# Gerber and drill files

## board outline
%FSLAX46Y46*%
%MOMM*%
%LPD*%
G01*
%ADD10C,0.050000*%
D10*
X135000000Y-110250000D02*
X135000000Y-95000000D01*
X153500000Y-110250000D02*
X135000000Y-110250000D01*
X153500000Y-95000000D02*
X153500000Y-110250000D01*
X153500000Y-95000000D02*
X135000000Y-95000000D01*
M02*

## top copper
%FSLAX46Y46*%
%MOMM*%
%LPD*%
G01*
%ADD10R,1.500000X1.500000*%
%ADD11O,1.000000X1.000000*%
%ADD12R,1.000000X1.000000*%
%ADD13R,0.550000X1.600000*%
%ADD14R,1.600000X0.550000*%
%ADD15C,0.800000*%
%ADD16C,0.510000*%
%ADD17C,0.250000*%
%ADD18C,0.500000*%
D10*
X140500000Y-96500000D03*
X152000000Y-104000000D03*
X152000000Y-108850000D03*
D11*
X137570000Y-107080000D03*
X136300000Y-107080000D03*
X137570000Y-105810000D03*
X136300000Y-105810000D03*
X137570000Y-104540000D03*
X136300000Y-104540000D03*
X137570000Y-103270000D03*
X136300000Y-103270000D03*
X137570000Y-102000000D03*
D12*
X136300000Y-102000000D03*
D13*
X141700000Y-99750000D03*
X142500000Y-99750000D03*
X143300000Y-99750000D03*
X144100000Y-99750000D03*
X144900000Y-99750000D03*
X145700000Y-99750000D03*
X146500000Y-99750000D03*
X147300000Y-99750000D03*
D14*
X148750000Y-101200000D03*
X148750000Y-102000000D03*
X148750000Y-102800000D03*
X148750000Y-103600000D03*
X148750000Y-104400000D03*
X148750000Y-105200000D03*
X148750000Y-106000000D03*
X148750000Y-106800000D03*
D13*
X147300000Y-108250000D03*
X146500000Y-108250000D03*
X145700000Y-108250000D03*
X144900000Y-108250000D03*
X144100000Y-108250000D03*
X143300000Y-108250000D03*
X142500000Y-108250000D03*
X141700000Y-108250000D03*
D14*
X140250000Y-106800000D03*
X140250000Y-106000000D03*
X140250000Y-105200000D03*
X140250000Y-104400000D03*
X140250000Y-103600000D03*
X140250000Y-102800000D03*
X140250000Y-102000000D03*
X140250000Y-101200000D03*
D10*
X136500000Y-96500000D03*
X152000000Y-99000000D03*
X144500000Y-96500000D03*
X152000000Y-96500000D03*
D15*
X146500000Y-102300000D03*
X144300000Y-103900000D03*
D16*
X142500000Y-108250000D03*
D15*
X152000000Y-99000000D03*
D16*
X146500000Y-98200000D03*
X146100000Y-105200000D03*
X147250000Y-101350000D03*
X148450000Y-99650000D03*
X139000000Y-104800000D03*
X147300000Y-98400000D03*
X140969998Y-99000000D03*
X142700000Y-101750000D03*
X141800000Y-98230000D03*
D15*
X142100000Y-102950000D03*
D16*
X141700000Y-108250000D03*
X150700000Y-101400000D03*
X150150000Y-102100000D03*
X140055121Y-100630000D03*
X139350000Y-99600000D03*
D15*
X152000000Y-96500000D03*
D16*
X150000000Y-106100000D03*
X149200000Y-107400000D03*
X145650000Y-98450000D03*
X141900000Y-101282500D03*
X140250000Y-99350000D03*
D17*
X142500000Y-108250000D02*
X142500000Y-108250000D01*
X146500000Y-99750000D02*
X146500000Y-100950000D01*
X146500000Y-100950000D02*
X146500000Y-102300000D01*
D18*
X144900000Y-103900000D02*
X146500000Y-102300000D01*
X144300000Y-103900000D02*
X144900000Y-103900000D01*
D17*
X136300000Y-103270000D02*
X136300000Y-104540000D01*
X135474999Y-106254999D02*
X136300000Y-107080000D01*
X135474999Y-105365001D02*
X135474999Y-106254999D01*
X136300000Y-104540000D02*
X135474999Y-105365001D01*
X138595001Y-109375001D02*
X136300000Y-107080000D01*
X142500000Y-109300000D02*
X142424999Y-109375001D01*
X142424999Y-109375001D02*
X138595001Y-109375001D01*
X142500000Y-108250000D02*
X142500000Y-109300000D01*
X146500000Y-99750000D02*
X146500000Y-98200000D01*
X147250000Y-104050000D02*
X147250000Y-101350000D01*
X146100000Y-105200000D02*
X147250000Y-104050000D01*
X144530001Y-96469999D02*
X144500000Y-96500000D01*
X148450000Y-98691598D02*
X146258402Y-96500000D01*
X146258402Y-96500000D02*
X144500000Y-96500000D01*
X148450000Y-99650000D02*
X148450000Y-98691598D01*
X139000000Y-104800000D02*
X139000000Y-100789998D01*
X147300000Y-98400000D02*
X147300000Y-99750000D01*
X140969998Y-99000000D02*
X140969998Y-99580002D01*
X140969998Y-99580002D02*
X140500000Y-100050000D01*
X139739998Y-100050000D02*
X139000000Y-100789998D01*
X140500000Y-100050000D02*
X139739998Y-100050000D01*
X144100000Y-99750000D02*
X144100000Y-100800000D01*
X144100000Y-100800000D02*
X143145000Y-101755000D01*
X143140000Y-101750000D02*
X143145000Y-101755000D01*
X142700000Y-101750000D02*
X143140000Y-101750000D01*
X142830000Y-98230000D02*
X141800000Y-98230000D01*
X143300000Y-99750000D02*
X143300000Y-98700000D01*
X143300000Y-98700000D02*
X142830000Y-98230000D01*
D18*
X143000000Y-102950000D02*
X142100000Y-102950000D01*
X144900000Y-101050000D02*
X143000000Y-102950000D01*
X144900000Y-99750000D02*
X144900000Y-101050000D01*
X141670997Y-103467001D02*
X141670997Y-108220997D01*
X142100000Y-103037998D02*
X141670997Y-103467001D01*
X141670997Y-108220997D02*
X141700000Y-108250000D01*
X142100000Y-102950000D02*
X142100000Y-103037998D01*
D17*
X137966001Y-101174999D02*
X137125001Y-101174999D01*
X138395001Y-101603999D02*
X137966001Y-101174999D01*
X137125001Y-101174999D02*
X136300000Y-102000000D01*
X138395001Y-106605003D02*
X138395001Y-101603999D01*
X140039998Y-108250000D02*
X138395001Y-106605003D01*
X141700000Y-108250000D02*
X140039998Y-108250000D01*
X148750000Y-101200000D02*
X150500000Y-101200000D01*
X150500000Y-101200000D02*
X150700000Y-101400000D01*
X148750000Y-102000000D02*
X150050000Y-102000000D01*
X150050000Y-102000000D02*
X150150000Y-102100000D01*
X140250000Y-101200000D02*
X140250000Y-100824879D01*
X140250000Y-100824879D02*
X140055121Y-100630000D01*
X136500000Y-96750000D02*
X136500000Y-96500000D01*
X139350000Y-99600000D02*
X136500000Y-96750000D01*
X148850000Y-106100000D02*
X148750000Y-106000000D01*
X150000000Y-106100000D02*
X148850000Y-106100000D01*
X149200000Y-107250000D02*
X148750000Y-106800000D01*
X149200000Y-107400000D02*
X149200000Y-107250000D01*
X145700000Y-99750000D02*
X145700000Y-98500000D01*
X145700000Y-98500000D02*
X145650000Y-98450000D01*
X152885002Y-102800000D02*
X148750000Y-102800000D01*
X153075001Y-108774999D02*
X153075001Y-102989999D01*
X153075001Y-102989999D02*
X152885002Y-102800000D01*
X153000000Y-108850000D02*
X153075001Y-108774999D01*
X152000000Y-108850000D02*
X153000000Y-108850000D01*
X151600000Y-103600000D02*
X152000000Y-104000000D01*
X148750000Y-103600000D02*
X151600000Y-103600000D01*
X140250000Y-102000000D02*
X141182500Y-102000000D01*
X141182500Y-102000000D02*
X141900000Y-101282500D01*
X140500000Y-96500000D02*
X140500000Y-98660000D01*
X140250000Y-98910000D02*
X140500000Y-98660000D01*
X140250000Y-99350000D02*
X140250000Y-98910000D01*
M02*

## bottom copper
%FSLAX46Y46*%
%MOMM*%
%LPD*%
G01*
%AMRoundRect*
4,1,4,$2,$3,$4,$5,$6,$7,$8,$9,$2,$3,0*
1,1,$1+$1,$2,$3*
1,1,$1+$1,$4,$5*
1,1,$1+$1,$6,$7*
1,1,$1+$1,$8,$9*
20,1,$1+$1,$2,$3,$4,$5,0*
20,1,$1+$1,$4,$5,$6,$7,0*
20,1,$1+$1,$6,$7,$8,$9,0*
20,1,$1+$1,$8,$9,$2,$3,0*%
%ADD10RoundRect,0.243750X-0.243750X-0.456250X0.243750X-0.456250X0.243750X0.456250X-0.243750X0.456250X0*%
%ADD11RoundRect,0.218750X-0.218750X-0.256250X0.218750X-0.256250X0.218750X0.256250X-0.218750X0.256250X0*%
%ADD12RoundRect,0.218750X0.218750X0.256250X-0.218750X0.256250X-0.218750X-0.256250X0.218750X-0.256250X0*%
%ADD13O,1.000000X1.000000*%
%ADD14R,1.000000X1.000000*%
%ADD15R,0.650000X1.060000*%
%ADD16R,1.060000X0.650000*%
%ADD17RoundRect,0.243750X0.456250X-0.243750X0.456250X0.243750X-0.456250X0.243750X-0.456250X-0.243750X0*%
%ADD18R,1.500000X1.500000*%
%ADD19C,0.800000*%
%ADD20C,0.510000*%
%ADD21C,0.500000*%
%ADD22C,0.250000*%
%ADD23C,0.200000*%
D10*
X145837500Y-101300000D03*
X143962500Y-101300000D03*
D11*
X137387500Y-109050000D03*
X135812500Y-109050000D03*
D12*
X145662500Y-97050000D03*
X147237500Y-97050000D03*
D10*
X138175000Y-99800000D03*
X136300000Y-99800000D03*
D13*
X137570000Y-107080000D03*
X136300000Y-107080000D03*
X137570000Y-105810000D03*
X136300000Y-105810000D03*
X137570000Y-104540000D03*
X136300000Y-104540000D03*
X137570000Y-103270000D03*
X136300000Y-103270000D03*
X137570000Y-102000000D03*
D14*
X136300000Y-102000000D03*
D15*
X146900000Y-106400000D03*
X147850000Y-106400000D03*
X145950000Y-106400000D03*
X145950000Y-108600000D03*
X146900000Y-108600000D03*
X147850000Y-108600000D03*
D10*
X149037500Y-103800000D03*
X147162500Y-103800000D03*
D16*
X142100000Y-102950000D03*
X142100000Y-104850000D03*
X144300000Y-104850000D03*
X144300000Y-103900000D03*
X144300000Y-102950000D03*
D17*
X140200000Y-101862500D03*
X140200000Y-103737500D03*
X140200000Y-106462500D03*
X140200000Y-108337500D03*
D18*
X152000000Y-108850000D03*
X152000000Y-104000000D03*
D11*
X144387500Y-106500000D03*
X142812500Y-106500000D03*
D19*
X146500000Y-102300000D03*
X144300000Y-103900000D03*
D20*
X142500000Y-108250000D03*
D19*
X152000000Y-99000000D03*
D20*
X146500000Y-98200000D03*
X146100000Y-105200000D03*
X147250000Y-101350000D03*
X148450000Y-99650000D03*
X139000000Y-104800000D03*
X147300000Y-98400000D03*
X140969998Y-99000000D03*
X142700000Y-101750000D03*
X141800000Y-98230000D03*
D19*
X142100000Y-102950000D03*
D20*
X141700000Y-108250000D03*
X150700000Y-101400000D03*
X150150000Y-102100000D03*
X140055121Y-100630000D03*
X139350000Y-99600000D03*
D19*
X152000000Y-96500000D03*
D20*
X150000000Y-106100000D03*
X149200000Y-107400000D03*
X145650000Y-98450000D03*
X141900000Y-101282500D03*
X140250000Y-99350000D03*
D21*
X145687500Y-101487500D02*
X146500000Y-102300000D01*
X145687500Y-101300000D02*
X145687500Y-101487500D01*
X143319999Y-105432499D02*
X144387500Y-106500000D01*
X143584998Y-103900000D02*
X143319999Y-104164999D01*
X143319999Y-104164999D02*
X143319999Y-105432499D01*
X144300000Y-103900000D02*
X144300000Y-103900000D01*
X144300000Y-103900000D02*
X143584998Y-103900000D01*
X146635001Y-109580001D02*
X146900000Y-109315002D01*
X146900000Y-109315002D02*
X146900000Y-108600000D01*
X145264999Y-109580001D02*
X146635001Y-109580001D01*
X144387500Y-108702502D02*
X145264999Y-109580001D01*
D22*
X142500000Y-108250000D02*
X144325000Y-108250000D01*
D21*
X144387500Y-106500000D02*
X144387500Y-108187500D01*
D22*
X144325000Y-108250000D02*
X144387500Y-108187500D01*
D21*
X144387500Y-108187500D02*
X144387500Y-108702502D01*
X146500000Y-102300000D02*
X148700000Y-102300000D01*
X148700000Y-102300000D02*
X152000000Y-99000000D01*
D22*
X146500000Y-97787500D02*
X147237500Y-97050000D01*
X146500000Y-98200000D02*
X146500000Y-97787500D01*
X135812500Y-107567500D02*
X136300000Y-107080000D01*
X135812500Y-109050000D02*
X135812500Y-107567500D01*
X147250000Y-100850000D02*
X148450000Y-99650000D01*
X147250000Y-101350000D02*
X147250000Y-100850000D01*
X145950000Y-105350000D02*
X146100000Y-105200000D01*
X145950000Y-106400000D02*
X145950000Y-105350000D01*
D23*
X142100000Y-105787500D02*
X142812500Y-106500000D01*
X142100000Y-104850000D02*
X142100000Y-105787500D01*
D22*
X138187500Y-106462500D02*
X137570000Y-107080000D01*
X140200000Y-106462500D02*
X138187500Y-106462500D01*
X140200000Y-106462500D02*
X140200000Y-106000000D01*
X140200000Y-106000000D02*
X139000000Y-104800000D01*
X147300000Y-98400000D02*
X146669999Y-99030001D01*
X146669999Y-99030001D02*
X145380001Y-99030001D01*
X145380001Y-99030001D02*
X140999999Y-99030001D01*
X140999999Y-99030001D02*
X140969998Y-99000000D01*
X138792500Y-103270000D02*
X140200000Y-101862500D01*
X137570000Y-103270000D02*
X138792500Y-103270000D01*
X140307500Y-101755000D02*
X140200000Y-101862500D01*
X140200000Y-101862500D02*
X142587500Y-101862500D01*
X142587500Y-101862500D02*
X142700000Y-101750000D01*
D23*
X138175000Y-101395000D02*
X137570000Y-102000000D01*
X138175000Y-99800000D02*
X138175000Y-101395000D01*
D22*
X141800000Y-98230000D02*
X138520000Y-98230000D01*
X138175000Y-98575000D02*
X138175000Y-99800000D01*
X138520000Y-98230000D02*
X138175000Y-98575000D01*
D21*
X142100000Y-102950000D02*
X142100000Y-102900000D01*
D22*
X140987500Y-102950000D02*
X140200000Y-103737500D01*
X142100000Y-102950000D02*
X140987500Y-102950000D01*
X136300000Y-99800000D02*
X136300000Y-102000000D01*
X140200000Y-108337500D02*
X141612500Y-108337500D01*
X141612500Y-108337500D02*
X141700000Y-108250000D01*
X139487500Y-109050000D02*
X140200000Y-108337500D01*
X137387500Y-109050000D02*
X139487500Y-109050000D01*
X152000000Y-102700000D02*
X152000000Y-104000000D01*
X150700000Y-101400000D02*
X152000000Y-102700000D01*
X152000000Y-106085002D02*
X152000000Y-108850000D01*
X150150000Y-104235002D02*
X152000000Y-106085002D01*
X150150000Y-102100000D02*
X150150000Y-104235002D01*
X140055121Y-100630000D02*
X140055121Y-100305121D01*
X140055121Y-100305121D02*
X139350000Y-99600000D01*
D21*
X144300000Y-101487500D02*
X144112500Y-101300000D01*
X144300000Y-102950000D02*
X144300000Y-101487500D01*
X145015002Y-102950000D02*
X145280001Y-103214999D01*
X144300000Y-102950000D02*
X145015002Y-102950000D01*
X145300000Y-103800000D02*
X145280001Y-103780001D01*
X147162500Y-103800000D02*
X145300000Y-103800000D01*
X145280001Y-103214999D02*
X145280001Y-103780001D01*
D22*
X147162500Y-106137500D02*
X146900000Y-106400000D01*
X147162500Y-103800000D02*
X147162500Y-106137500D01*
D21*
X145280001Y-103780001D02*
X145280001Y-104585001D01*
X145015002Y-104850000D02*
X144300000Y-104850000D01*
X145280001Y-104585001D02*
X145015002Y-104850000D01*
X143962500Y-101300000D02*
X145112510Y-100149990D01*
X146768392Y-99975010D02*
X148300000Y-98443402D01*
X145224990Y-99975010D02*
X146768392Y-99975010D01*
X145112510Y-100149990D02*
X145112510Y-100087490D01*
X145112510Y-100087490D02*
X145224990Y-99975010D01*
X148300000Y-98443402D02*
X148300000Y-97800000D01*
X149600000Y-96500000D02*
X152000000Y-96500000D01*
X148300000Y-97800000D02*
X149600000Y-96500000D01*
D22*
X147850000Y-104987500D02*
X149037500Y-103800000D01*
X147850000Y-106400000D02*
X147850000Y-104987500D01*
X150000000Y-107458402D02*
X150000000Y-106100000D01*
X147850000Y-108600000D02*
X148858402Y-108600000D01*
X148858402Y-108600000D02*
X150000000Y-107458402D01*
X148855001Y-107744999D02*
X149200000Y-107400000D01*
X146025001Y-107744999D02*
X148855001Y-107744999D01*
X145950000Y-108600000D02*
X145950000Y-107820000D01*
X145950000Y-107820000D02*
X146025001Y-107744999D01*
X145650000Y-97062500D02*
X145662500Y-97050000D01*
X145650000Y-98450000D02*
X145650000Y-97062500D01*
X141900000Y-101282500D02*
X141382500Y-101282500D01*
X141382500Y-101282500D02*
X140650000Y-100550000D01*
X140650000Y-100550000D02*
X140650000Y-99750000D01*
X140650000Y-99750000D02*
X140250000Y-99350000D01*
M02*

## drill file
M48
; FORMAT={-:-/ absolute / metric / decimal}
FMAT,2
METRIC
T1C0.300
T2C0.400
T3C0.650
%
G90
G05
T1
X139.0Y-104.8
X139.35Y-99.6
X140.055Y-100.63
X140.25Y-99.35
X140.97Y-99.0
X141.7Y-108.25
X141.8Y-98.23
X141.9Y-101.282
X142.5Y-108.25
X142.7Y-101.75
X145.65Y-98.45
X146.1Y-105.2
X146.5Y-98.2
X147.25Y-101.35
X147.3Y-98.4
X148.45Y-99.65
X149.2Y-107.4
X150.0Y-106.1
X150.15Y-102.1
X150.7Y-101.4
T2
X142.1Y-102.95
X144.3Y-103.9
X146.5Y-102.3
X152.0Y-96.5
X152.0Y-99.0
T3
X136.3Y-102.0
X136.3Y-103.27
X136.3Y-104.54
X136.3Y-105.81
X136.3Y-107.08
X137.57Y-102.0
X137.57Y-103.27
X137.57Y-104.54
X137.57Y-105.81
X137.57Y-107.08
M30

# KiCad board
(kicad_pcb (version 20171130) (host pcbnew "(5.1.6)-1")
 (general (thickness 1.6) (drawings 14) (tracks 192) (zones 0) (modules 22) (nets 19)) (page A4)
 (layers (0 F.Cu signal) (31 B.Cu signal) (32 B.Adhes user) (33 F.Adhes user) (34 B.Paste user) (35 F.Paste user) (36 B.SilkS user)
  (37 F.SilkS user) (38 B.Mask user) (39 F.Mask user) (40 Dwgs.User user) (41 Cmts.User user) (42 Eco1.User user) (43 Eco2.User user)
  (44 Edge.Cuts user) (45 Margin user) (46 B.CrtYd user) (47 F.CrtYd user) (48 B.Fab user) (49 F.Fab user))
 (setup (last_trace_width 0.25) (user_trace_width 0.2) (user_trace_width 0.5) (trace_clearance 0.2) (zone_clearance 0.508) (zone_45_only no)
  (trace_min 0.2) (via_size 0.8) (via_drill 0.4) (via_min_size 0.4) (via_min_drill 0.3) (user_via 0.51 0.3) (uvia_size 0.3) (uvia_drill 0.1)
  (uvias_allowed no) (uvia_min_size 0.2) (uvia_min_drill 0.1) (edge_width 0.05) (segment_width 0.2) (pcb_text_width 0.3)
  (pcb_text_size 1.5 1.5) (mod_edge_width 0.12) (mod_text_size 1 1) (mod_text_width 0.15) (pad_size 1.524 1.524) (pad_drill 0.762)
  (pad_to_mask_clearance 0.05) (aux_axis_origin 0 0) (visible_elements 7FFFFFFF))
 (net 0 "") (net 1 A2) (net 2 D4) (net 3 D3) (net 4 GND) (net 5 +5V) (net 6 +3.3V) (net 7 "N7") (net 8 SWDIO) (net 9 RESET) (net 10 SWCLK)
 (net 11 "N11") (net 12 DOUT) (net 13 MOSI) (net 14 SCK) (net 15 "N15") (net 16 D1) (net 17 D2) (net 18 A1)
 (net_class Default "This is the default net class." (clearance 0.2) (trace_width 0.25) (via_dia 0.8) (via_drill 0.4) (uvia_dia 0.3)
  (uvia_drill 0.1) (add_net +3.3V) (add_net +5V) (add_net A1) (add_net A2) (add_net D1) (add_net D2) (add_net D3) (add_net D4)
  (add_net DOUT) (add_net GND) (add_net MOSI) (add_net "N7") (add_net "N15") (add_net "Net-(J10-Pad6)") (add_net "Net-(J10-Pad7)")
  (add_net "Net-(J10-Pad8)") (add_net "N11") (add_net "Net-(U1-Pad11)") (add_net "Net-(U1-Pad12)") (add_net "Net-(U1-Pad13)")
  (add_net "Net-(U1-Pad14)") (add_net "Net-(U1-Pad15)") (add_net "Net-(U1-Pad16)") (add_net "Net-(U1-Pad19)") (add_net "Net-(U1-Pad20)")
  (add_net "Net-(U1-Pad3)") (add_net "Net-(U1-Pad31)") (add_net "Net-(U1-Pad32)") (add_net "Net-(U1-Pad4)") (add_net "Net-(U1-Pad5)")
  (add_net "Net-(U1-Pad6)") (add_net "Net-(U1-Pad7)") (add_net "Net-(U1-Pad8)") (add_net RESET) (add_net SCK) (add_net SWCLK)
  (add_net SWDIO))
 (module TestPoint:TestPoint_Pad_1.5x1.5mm (layer F.Cu) (at 140.5 96.5)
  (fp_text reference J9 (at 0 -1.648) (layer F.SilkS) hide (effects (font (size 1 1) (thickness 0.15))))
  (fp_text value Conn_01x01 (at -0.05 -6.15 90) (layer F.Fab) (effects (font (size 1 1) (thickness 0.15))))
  (pad 1 smd rect (at 0 0) (size 1.5 1.5) (layers F.Cu F.Mask) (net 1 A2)))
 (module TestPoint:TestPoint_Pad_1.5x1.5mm (layer F.Cu) (at 152 104)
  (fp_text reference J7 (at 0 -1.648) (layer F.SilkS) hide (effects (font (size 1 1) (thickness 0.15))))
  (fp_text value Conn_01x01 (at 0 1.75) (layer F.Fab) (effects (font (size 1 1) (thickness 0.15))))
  (pad 1 smd rect (at 0 0) (size 1.5 1.5) (layers F.Cu F.Mask) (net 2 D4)))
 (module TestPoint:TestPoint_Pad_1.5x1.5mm (layer F.Cu) (at 152 108.85)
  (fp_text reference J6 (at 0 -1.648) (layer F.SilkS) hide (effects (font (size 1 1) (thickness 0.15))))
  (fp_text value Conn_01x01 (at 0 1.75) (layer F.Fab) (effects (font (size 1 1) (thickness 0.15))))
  (pad 1 smd rect (at 0 0) (size 1.5 1.5) (layers F.Cu F.Mask) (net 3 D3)))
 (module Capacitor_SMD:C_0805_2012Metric (layer B.Cu) (at 144.9 101.3)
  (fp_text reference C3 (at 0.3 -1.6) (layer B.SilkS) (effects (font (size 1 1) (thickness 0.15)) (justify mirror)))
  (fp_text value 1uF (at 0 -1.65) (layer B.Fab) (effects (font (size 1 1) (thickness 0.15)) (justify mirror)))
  (pad 2 smd roundrect (at 0.9375 0) (size 0.975 1.4) (layers B.Cu B.Paste B.Mask) (roundrect_rratio 0.25) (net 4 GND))
  (pad 1 smd roundrect (at -0.9375 0) (size 0.975 1.4) (layers B.Cu B.Paste B.Mask) (roundrect_rratio 0.25) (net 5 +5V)))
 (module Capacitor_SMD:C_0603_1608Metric (layer B.Cu) (at 136.6 109.05)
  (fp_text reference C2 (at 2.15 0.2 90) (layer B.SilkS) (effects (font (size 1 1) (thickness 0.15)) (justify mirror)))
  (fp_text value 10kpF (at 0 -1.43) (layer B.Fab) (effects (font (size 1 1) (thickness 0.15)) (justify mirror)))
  (pad 2 smd roundrect (at 0.7875 0) (size 0.875 0.95) (layers B.Cu B.Paste B.Mask) (roundrect_rratio 0.25) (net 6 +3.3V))
  (pad 1 smd roundrect (at -0.7875 0) (size 0.875 0.95) (layers B.Cu B.Paste B.Mask) (roundrect_rratio 0.25) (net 4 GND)))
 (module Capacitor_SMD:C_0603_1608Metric (layer B.Cu) (at 146.45 97.05 180)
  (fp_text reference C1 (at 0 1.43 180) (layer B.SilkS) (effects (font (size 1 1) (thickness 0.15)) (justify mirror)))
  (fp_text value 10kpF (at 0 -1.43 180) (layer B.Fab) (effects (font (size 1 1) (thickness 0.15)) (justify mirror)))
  (pad 2 smd roundrect (at 0.7875 0 180) (size 0.875 0.95) (layers B.Cu B.Paste B.Mask) (roundrect_rratio 0.25) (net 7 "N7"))
  (pad 1 smd roundrect (at -0.7875 0 180) (size 0.875 0.95) (layers B.Cu B.Paste B.Mask) (roundrect_rratio 0.25) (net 4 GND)))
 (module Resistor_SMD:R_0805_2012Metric (layer B.Cu) (at 137.2375 99.8)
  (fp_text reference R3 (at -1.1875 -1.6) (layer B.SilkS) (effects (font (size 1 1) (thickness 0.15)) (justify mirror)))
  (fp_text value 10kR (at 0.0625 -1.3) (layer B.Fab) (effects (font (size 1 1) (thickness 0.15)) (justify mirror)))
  (pad 2 smd roundrect (at 0.9375 0) (size 0.975 1.4) (layers B.Cu B.Paste B.Mask) (roundrect_rratio 0.25) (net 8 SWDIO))
  (pad 1 smd roundrect (at -0.9375 0) (size 0.975 1.4) (layers B.Cu B.Paste B.Mask) (roundrect_rratio 0.25) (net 6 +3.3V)))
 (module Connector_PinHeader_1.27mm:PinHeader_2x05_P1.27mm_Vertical (layer F.Cu) (at 136.3 102)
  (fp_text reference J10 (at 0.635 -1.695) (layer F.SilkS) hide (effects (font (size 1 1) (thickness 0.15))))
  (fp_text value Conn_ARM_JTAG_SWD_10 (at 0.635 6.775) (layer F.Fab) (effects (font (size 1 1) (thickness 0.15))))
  (pad 10 thru_hole oval (at 1.27 5.08) (size 1 1) (drill 0.65) (layers *.Cu *.Mask) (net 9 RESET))
  (pad 9 thru_hole oval (at 0 5.08) (size 1 1) (drill 0.65) (layers *.Cu *.Mask) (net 4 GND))
  (pad 8 thru_hole oval (at 1.27 3.81) (size 1 1) (drill 0.65) (layers *.Cu *.Mask))
  (pad 7 thru_hole oval (at 0 3.81) (size 1 1) (drill 0.65) (layers *.Cu *.Mask))
  (pad 6 thru_hole oval (at 1.27 2.54) (size 1 1) (drill 0.65) (layers *.Cu *.Mask))
  (pad 5 thru_hole oval (at 0 2.54) (size 1 1) (drill 0.65) (layers *.Cu *.Mask) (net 4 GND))
  (pad 4 thru_hole oval (at 1.27 1.27) (size 1 1) (drill 0.65) (layers *.Cu *.Mask) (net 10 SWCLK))
  (pad 3 thru_hole oval (at 0 1.27) (size 1 1) (drill 0.65) (layers *.Cu *.Mask) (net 4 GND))
  (pad 2 thru_hole oval (at 1.27 0) (size 1 1) (drill 0.65) (layers *.Cu *.Mask) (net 8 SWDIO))
  (pad 1 thru_hole rect (at 0 0) (size 1 1) (drill 0.65) (layers *.Cu *.Mask) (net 6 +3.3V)))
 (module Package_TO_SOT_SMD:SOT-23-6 (layer B.Cu) (at 146.9 107.5 90)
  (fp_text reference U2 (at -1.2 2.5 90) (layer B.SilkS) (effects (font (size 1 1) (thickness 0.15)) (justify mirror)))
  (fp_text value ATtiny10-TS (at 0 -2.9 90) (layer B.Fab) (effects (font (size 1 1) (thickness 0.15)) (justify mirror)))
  (pad 5 smd rect (at 1.1 0 90) (size 1.06 0.65) (layers B.Cu B.Paste B.Mask) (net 5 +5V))
  (pad 6 smd rect (at 1.1 0.95 90) (size 1.06 0.65) (layers B.Cu B.Paste B.Mask) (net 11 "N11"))
  (pad 4 smd rect (at 1.1 -0.95 90) (size 1.06 0.65) (layers B.Cu B.Paste B.Mask) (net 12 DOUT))
  (pad 3 smd rect (at -1.1 -0.95 90) (size 1.06 0.65) (layers B.Cu B.Paste B.Mask) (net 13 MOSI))
  (pad 2 smd rect (at -1.1 0 90) (size 1.06 0.65) (layers B.Cu B.Paste B.Mask) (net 4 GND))
  (pad 1 smd rect (at -1.1 0.95 90) (size 1.06 0.65) (layers B.Cu B.Paste B.Mask) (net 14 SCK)))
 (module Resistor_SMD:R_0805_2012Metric (layer B.Cu) (at 148.1 103.8)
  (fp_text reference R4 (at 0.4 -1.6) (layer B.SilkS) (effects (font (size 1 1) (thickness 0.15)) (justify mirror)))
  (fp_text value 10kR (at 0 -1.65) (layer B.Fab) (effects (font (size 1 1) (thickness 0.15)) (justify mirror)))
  (pad 2 smd roundrect (at 0.9375 0) (size 0.975 1.4) (layers B.Cu B.Paste B.Mask) (roundrect_rratio 0.25) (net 11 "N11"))
  (pad 1 smd roundrect (at -0.9375 0) (size 0.975 1.4) (layers B.Cu B.Paste B.Mask) (roundrect_rratio 0.25) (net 5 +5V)))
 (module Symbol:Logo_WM (layer F.Cu) (at 137.8 99.1)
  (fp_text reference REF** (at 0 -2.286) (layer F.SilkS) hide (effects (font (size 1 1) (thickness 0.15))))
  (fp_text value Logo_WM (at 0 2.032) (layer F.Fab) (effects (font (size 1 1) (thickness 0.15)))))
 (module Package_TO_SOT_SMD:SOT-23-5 (layer B.Cu) (at 143.2 103.9 180)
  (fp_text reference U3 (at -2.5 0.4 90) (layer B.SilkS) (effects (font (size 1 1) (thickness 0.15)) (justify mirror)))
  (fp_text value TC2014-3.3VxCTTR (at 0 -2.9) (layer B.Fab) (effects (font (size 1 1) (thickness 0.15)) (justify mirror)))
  (pad 5 smd rect (at 1.1 0.95 180) (size 1.06 0.65) (layers B.Cu B.Paste B.Mask) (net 6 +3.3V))
  (pad 4 smd rect (at 1.1 -0.95 180) (size 1.06 0.65) (layers B.Cu B.Paste B.Mask) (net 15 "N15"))
  (pad 3 smd rect (at -1.1 -0.95 180) (size 1.06 0.65) (layers B.Cu B.Paste B.Mask) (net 5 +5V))
  (pad 2 smd rect (at -1.1 0 180) (size 1.06 0.65) (layers B.Cu B.Paste B.Mask) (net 4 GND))
  (pad 1 smd rect (at -1.1 0.95 180) (size 1.06 0.65) (layers B.Cu B.Paste B.Mask) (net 5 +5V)))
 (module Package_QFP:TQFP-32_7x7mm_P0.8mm (layer F.Cu) (at 144.5 104)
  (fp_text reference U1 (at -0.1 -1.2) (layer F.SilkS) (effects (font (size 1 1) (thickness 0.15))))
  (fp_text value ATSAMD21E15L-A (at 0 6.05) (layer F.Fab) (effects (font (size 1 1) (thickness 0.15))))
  (pad 32 smd rect (at -2.8 -4.25 90) (size 1.6 0.55) (layers F.Cu F.Paste F.Mask))
  (pad 31 smd rect (at -2 -4.25 90) (size 1.6 0.55) (layers F.Cu F.Paste F.Mask))
  (pad 30 smd rect (at -1.2 -4.25 90) (size 1.6 0.55) (layers F.Cu F.Paste F.Mask) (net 8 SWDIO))
  (pad 29 smd rect (at -0.4 -4.25 90) (size 1.6 0.55) (layers F.Cu F.Paste F.Mask) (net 10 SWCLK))
  (pad 28 smd rect (at 0.4 -4.25 90) (size 1.6 0.55) (layers F.Cu F.Paste F.Mask) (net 6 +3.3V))
  (pad 27 smd rect (at 1.2 -4.25 90) (size 1.6 0.55) (layers F.Cu F.Paste F.Mask) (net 7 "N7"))
  (pad 26 smd rect (at 2 -4.25 90) (size 1.6 0.55) (layers F.Cu F.Paste F.Mask) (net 4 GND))
  (pad 25 smd rect (at 2.8 -4.25 90) (size 1.6 0.55) (layers F.Cu F.Paste F.Mask) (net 9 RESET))
  (pad 24 smd rect (at 4.25 -2.8) (size 1.6 0.55) (layers F.Cu F.Paste F.Mask) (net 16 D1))
  (pad 23 smd rect (at 4.25 -2) (size 1.6 0.55) (layers F.Cu F.Paste F.Mask) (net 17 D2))
  (pad 22 smd rect (at 4.25 -1.2) (size 1.6 0.55) (layers F.Cu F.Paste F.Mask) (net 3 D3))
  (pad 21 smd rect (at 4.25 -0.4) (size 1.6 0.55) (layers F.Cu F.Paste F.Mask) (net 2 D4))
  (pad 20 smd rect (at 4.25 0.4) (size 1.6 0.55) (layers F.Cu F.Paste F.Mask))
  (pad 19 smd rect (at 4.25 1.2) (size 1.6 0.55) (layers F.Cu F.Paste F.Mask))
  (pad 18 smd rect (at 4.25 2) (size 1.6 0.55) (layers F.Cu F.Paste F.Mask) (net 14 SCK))
  (pad 17 smd rect (at 4.25 2.8) (size 1.6 0.55) (layers F.Cu F.Paste F.Mask) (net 13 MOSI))
  (pad 16 smd rect (at 2.8 4.25 90) (size 1.6 0.55) (layers F.Cu F.Paste F.Mask))
  (pad 15 smd rect (at 2 4.25 90) (size 1.6 0.55) (layers F.Cu F.Paste F.Mask))
  (pad 14 smd rect (at 1.2 4.25 90) (size 1.6 0.55) (layers F.Cu F.Paste F.Mask))
  (pad 13 smd rect (at 0.4 4.25 90) (size 1.6 0.55) (layers F.Cu F.Paste F.Mask))
  (pad 12 smd rect (at -0.4 4.25 90) (size 1.6 0.55) (layers F.Cu F.Paste F.Mask))
  (pad 11 smd rect (at -1.2 4.25 90) (size 1.6 0.55) (layers F.Cu F.Paste F.Mask))
  (pad 10 smd rect (at -2 4.25 90) (size 1.6 0.55) (layers F.Cu F.Paste F.Mask) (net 4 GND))
  (pad 9 smd rect (at -2.8 4.25 90) (size 1.6 0.55) (layers F.Cu F.Paste F.Mask) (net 6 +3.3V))
  (pad 8 smd rect (at -4.25 2.8) (size 1.6 0.55) (layers F.Cu F.Paste F.Mask))
  (pad 7 smd rect (at -4.25 2) (size 1.6 0.55) (layers F.Cu F.Paste F.Mask))
  (pad 6 smd rect (at -4.25 1.2) (size 1.6 0.55) (layers F.Cu F.Paste F.Mask))
  (pad 5 smd rect (at -4.25 0.4) (size 1.6 0.55) (layers F.Cu F.Paste F.Mask))
  (pad 4 smd rect (at -4.25 -0.4) (size 1.6 0.55) (layers F.Cu F.Paste F.Mask))
  (pad 3 smd rect (at -4.25 -1.2) (size 1.6 0.55) (layers F.Cu F.Paste F.Mask))
  (pad 2 smd rect (at -4.25 -2) (size 1.6 0.55) (layers F.Cu F.Paste F.Mask) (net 1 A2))
  (pad 1 smd rect (at -4.25 -2.8) (size 1.6 0.55) (layers F.Cu F.Paste F.Mask) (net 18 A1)))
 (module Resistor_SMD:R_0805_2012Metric (layer B.Cu) (at 140.2 102.8 90)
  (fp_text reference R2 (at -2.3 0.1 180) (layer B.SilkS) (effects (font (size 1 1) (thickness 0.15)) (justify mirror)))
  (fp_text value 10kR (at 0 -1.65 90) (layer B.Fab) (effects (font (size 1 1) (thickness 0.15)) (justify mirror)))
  (pad 2 smd roundrect (at 0.9375 0 90) (size 0.975 1.4) (layers B.Cu B.Paste B.Mask) (roundrect_rratio 0.25) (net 10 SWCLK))
  (pad 1 smd roundrect (at -0.9375 0 90) (size 0.975 1.4) (layers B.Cu B.Paste B.Mask) (roundrect_rratio 0.25) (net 6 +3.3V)))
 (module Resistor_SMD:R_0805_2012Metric (layer B.Cu) (at 140.2 107.4 90)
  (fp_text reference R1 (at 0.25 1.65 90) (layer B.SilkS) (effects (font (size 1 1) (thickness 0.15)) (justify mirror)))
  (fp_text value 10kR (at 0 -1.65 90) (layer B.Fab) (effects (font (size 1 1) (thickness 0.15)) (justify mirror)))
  (pad 2 smd roundrect (at 0.9375 0 90) (size 0.975 1.4) (layers B.Cu B.Paste B.Mask) (roundrect_rratio 0.25) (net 9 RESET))
  (pad 1 smd roundrect (at -0.9375 0 90) (size 0.975 1.4) (layers B.Cu B.Paste B.Mask) (roundrect_rratio 0.25) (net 6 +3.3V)))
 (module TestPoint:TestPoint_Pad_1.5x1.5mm (layer F.Cu) (at 136.5 96.5)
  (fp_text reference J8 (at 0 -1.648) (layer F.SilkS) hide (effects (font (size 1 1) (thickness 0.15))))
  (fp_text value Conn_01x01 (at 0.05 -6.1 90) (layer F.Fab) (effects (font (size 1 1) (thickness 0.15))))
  (pad 1 smd rect (at 0 0) (size 1.5 1.5) (layers F.Cu F.Mask) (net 18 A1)))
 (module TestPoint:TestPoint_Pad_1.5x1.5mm (layer B.Cu) (at 152 108.85)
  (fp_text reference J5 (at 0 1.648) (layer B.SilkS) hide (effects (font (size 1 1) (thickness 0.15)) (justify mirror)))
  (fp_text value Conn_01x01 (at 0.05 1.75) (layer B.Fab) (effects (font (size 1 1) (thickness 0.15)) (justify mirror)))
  (pad 1 smd rect (at 0 0) (size 1.5 1.5) (layers B.Cu B.Mask) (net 17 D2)))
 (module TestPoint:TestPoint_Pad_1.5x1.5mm (layer B.Cu) (at 152 104)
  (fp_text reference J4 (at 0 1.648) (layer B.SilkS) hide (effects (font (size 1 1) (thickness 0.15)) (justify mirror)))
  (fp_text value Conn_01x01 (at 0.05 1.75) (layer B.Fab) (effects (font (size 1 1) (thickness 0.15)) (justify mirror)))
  (pad 1 smd rect (at 0 0) (size 1.5 1.5) (layers B.Cu B.Mask) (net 16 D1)))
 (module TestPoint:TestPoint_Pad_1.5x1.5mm (layer F.Cu) (at 152 99)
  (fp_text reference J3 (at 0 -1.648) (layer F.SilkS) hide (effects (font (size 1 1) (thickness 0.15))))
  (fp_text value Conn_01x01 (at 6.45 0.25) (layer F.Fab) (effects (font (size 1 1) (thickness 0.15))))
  (pad 1 smd rect (at 0 0) (size 1.5 1.5) (layers F.Cu F.Mask) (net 4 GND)))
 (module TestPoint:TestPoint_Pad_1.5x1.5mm (layer F.Cu) (at 144.5 96.5)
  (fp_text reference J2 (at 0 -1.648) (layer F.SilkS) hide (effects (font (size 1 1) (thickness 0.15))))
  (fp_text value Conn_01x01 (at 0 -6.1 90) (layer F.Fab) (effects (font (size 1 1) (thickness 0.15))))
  (pad 1 smd rect (at 0 0) (size 1.5 1.5) (layers F.Cu F.Mask) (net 12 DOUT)))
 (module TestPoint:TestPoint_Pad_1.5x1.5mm (layer F.Cu) (at 152 96.5)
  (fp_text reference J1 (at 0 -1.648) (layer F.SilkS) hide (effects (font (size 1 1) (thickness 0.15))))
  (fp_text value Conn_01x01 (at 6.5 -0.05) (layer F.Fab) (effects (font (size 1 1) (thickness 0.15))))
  (pad 1 smd rect (at 0 0) (size 1.5 1.5) (layers F.Cu F.Mask) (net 5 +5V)))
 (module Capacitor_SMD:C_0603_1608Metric (layer B.Cu) (at 143.6 106.5)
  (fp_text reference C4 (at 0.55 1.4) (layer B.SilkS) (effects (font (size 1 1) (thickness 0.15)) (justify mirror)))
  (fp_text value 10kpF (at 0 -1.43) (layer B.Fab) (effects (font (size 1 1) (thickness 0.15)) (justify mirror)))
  (pad 2 smd roundrect (at 0.7875 0) (size 0.875 0.95) (layers B.Cu B.Paste B.Mask) (roundrect_rratio 0.25) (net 4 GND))
  (pad 1 smd roundrect (at -0.7875 0) (size 0.875 0.95) (layers B.Cu B.Paste B.Mask) (roundrect_rratio 0.25) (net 15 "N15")))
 (gr_line (start 135 110.25) (end 135 95) (layer Edge.Cuts) (width 0.05))
 (gr_line (start 153.5 110.25) (end 135 110.25) (layer Edge.Cuts) (width 0.05))
 (gr_line (start 153.5 95) (end 153.5 110.25) (layer Edge.Cuts) (width 0.05))
 (gr_line (start 153.5 95) (end 135 95) (layer Edge.Cuts) (width 0.05))
 (segment (start 142.5 108.25) (end 142.5 108.25) (width 0.25) (layer F.Cu) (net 4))
 (segment (start 146.5 99.75) (end 146.5 100.95) (width 0.25) (layer F.Cu) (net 4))
 (segment (start 145.6875 101.4875) (end 146.5 102.3) (width 0.5) (layer B.Cu) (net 4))
 (segment (start 145.6875 101.3) (end 145.6875 101.4875) (width 0.5) (layer B.Cu) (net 4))
 (via (at 146.5 102.3) (size 0.8) (drill 0.4) (layers F.Cu B.Cu) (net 4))
 (segment (start 146.5 100.95) (end 146.5 102.3) (width 0.25) (layer F.Cu) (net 4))
 (segment (start 143.319999 105.432499) (end 144.3875 106.5) (width 0.5) (layer B.Cu) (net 4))
 (segment (start 143.584998 103.9) (end 143.319999 104.164999) (width 0.5) (layer B.Cu) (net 4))
 (segment (start 143.319999 104.164999) (end 143.319999 105.432499) (width 0.5) (layer B.Cu) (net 4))
 (segment (start 144.3 103.9) (end 144.3 103.9) (width 0.5) (layer B.Cu) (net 4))
 (segment (start 144.3 103.9) (end 143.584998 103.9) (width 0.5) (layer B.Cu) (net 4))
 (via (at 144.3 103.9) (size 0.8) (drill 0.4) (layers F.Cu B.Cu) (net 4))
 (segment (start 144.9 103.9) (end 146.5 102.3) (width 0.5) (layer F.Cu) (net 4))
 (segment (start 144.3 103.9) (end 144.9 103.9) (width 0.5) (layer F.Cu) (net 4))
 (segment (start 146.635001 109.580001) (end 146.9 109.315002) (width 0.5) (layer B.Cu) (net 4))
 (segment (start 146.9 109.315002) (end 146.9 108.6) (width 0.5) (layer B.Cu) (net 4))
 (segment (start 145.264999 109.580001) (end 146.635001 109.580001) (width 0.5) (layer B.Cu) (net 4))
 (segment (start 144.3875 108.702502) (end 145.264999 109.580001) (width 0.5) (layer B.Cu) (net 4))
 (via (at 142.5 108.25) (size 0.51) (drill 0.3) (layers F.Cu B.Cu) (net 4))
 (segment (start 142.5 108.25) (end 144.325 108.25) (width 0.25) (layer B.Cu) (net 4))
 (segment (start 144.3875 106.5) (end 144.3875 108.1875) (width 0.5) (layer B.Cu) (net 4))
 (segment (start 144.325 108.25) (end 144.3875 108.1875) (width 0.25) (layer B.Cu) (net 4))
 (segment (start 144.3875 108.1875) (end 144.3875 108.702502) (width 0.5) (layer B.Cu) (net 4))
 (segment (start 136.3 103.27) (end 136.3 104.54) (width 0.25) (layer F.Cu) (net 4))
 (segment (start 135.474999 106.254999) (end 136.3 107.08) (width 0.25) (layer F.Cu) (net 4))
 (segment (start 135.474999 105.365001) (end 135.474999 106.254999) (width 0.25) (layer F.Cu) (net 4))
 (segment (start 136.3 104.54) (end 135.474999 105.365001) (width 0.25) (layer F.Cu) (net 4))
 (segment (start 138.595001 109.375001) (end 136.3 107.08) (width 0.25) (layer F.Cu) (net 4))
 (segment (start 142.5 109.3) (end 142.424999 109.375001) (width 0.25) (layer F.Cu) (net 4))
 (segment (start 142.424999 109.375001) (end 138.595001 109.375001) (width 0.25) (layer F.Cu) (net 4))
 (segment (start 142.5 108.25) (end 142.5 109.3) (width 0.25) (layer F.Cu) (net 4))
 (via (at 152 99) (size 0.8) (drill 0.4) (layers F.Cu B.Cu) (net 4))
 (segment (start 146.5 102.3) (end 148.7 102.3) (width 0.5) (layer B.Cu) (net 4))
 (segment (start 148.7 102.3) (end 152 99) (width 0.5) (layer B.Cu) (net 4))
 (via (at 146.5 98.2) (size 0.51) (drill 0.3) (layers F.Cu B.Cu) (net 4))
 (segment (start 146.5 99.75) (end 146.5 98.2) (width 0.25) (layer F.Cu) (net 4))
 (segment (start 146.5 97.7875) (end 147.2375 97.05) (width 0.25) (layer B.Cu) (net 4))
 (segment (start 146.5 98.2) (end 146.5 97.7875) (width 0.25) (layer B.Cu) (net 4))
 (segment (start 135.8125 107.5675) (end 136.3 107.08) (width 0.25) (layer B.Cu) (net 4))
 (segment (start 135.8125 109.05) (end 135.8125 107.5675) (width 0.25) (layer B.Cu) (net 4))
 (via (at 146.1 105.2) (size 0.51) (drill 0.3) (layers F.Cu B.Cu) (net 12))
 (via (at 147.25 101.35) (size 0.51) (drill 0.3) (layers F.Cu B.Cu) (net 12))
 (via (at 148.45 99.65) (size 0.51) (drill 0.3) (layers F.Cu B.Cu) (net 12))
 (segment (start 147.25 104.05) (end 147.25 101.35) (width 0.25) (layer F.Cu) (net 12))
 (segment (start 147.25 100.85) (end 148.45 99.65) (width 0.25) (layer B.Cu) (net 12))
 (segment (start 147.25 101.35) (end 147.25 100.85) (width 0.25) (layer B.Cu) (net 12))
 (segment (start 146.1 105.2) (end 147.25 104.05) (width 0.25) (layer F.Cu) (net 12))
 (segment (start 144.530001 96.469999) (end 144.5 96.5) (width 0.25) (layer F.Cu) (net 12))
 (segment (start 145.95 105.35) (end 146.1 105.2) (width 0.25) (layer B.Cu) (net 12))
 (segment (start 145.95 106.4) (end 145.95 105.35) (width 0.25) (layer B.Cu) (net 12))
 (segment (start 148.45 98.691598) (end 146.258402 96.5) (width 0.25) (layer F.Cu) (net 12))
 (segment (start 146.258402 96.5) (end 144.5 96.5) (width 0.25) (layer F.Cu) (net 12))
 (segment (start 148.45 99.65) (end 148.45 98.691598) (width 0.25) (layer F.Cu) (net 12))
 (segment (start 142.1 105.7875) (end 142.8125 106.5) (width 0.2) (layer B.Cu) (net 15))
 (segment (start 142.1 104.85) (end 142.1 105.7875) (width 0.2) (layer B.Cu) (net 15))
 (segment (start 138.1875 106.4625) (end 137.57 107.08) (width 0.25) (layer B.Cu) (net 9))
 (segment (start 140.2 106.4625) (end 138.1875 106.4625) (width 0.25) (layer B.Cu) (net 9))
 (via (at 139 104.8) (size 0.51) (drill 0.3) (layers F.Cu B.Cu) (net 9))
 (segment (start 140.2 106.4625) (end 140.2 106) (width 0.25) (layer B.Cu) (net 9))
 (segment (start 140.2 106) (end 139 104.8) (width 0.25) (layer B.Cu) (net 9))
 (segment (start 139 104.8) (end 139 100.789998) (width 0.25) (layer F.Cu) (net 9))
 (via (at 147.3 98.4) (size 0.51) (drill 0.3) (layers F.Cu B.Cu) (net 9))
 (segment (start 147.3 98.4) (end 147.3 99.75) (width 0.25) (layer F.Cu) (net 9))
 (segment (start 147.3 98.4) (end 146.669999 99.030001) (width 0.25) (layer B.Cu) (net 9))
 (segment (start 146.669999 99.030001) (end 145.380001 99.030001) (width 0.25) (layer B.Cu) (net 9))
 (segment (start 145.380001 99.030001) (end 140.999999 99.030001) (width 0.25) (layer B.Cu) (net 9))
 (via (at 140.969998 99) (size 0.51) (drill 0.3) (layers F.Cu B.Cu) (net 9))
 (segment (start 140.999999 99.030001) (end 140.969998 99) (width 0.25) (layer B.Cu) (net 9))
 (segment (start 140.969998 99) (end 140.969998 99.580002) (width 0.25) (layer F.Cu) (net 9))
 (segment (start 140.969998 99.580002) (end 140.5 100.05) (width 0.25) (layer F.Cu) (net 9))
 (segment (start 139.739998 100.05) (end 139 100.789998) (width 0.25) (layer F.Cu) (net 9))
 (segment (start 140.5 100.05) (end 139.739998 100.05) (width 0.25) (layer F.Cu) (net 9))
 (segment (start 138.7925 103.27) (end 140.2 101.8625) (width 0.25) (layer B.Cu) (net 10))
 (segment (start 137.57 103.27) (end 138.7925 103.27) (width 0.25) (layer B.Cu) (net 10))
 (segment (start 144.1 99.75) (end 144.1 100.8) (width 0.25) (layer F.Cu) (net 10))
 (segment (start 144.1 100.8) (end 143.145 101.755) (width 0.25) (layer F.Cu) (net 10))
 (segment (start 140.3075 101.755) (end 140.2 101.8625) (width 0.25) (layer B.Cu) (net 10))
 (via (at 142.7 101.75) (size 0.51) (drill 0.3) (layers F.Cu B.Cu) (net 10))
 (segment (start 140.2 101.8625) (end 142.5875 101.8625) (width 0.25) (layer B.Cu) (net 10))
 (segment (start 142.5875 101.8625) (end 142.7 101.75) (width 0.25) (layer B.Cu) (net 10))
 (segment (start 143.14 101.75) (end 143.145 101.755) (width 0.25) (layer F.Cu) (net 10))
 (segment (start 142.7 101.75) (end 143.14 101.75) (width 0.25) (layer F.Cu) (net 10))
 (segment (start 138.175 101.395) (end 137.57 102) (width 0.2) (layer B.Cu) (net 8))
 (segment (start 138.175 99.8) (end 138.175 101.395) (width 0.2) (layer B.Cu) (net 8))
 (segment (start 142.83 98.23) (end 141.8 98.23) (width 0.25) (layer F.Cu) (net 8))
 (segment (start 143.3 99.75) (end 143.3 98.7) (width 0.25) (layer F.Cu) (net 8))
 (via (at 141.8 98.23) (size 0.51) (drill 0.3) (layers F.Cu B.Cu) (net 8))
 (segment (start 143.3 98.7) (end 142.83 98.23) (width 0.25) (layer F.Cu) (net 8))
 (segment (start 141.8 98.23) (end 138.52 98.23) (width 0.25) (layer B.Cu) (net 8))
 (segment (start 138.175 98.575) (end 138.175 99.8) (width 0.25) (layer B.Cu) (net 8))
 (segment (start 138.52 98.23) (end 138.175 98.575) (width 0.25) (layer B.Cu) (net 8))
 (segment (start 143 102.95) (end 142.1 102.95) (width 0.5) (layer F.Cu) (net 6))
 (via (at 142.1 102.95) (size 0.8) (drill 0.4) (layers F.Cu B.Cu) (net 6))
 (segment (start 144.9 101.05) (end 143 102.95) (width 0.5) (layer F.Cu) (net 6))
 (segment (start 144.9 99.75) (end 144.9 101.05) (width 0.5) (layer F.Cu) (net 6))
 (segment (start 141.670997 103.467001) (end 141.670997 108.220997) (width 0.5) (layer F.Cu) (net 6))
 (segment (start 142.1 103.037998) (end 141.670997 103.467001) (width 0.5) (layer F.Cu) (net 6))
 (segment (start 141.670997 108.220997) (end 141.7 108.25) (width 0.5) (layer F.Cu) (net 6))
 (segment (start 142.1 102.95) (end 142.1 103.037998) (width 0.5) (layer F.Cu) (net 6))
 (segment (start 142.1 102.95) (end 142.1 102.9) (width 0.5) (layer B.Cu) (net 6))
 (segment (start 140.9875 102.95) (end 140.2 103.7375) (width 0.25) (layer B.Cu) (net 6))
 (segment (start 142.1 102.95) (end 140.9875 102.95) (width 0.25) (layer B.Cu) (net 6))
 (segment (start 136.3 99.8) (end 136.3 102) (width 0.25) (layer B.Cu) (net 6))
 (via (at 141.7 108.25) (size 0.51) (drill 0.3) (layers F.Cu B.Cu) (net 6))
 (segment (start 140.2 108.3375) (end 141.6125 108.3375) (width 0.25) (layer B.Cu) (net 6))
 (segment (start 141.6125 108.3375) (end 141.7 108.25) (width 0.25) (layer B.Cu) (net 6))
 (segment (start 137.966001 101.174999) (end 137.125001 101.174999) (width 0.25) (layer F.Cu) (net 6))
 (segment (start 138.395001 101.603999) (end 137.966001 101.174999) (width 0.25) (layer F.Cu) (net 6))
 (segment (start 137.125001 101.174999) (end 136.3 102) (width 0.25) (layer F.Cu) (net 6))
 (segment (start 138.395001 106.605003) (end 138.395001 101.603999) (width 0.25) (layer F.Cu) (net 6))
 (segment (start 140.039998 108.25) (end 138.395001 106.605003) (width 0.25) (layer F.Cu) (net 6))
 (segment (start 141.7 108.25) (end 140.039998 108.25) (width 0.25) (layer F.Cu) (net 6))
 (segment (start 139.4875 109.05) (end 140.2 108.3375) (width 0.25) (layer B.Cu) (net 6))
 (segment (start 137.3875 109.05) (end 139.4875 109.05) (width 0.25) (layer B.Cu) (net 6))
 (segment (start 148.75 101.2) (end 150.5 101.2) (width 0.25) (layer F.Cu) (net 16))
 (via (at 150.7 101.4) (size 0.51) (drill 0.3) (layers F.Cu B.Cu) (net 16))
 (segment (start 150.5 101.2) (end 150.7 101.4) (width 0.25) (layer F.Cu) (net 16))
 (segment (start 152 102.7) (end 152 104) (width 0.25) (layer B.Cu) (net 16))
 (segment (start 150.7 101.4) (end 152 102.7) (width 0.25) (layer B.Cu) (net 16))
 (via (at 150.15 102.1) (size 0.51) (drill 0.3) (layers F.Cu B.Cu) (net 17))
 (segment (start 148.75 102) (end 150.05 102) (width 0.25) (layer F.Cu) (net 17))
 (segment (start 150.05 102) (end 150.15 102.1) (width 0.25) (layer F.Cu) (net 17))
 (segment (start 152 106.085002) (end 152 108.85) (width 0.25) (layer B.Cu) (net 17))
 (segment (start 150.15 104.235002) (end 152 106.085002) (width 0.25) (layer B.Cu) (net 17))
 (segment (start 150.15 102.1) (end 150.15 104.235002) (width 0.25) (layer B.Cu) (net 17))
 (via (at 140.055121 100.63) (size 0.51) (drill 0.3) (layers F.Cu B.Cu) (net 18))
 (segment (start 140.25 101.2) (end 140.25 100.824879) (width 0.25) (layer F.Cu) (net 18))
 (segment (start 140.25 100.824879) (end 140.055121 100.63) (width 0.25) (layer F.Cu) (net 18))
 (via (at 139.35 99.6) (size 0.51) (drill 0.3) (layers F.Cu B.Cu) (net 18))
 (segment (start 140.055121 100.63) (end 140.055121 100.305121) (width 0.25) (layer B.Cu) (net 18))
 (segment (start 140.055121 100.305121) (end 139.35 99.6) (width 0.25) (layer B.Cu) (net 18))
 (segment (start 136.5 96.75) (end 136.5 96.5) (width 0.25) (layer F.Cu) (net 18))
 (segment (start 139.35 99.6) (end 136.5 96.75) (width 0.25) (layer F.Cu) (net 18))
 (segment (start 144.3 101.4875) (end 144.1125 101.3) (width 0.5) (layer B.Cu) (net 5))
 (segment (start 144.3 102.95) (end 144.3 101.4875) (width 0.5) (layer B.Cu) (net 5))
 (segment (start 145.015002 102.95) (end 145.280001 103.214999) (width 0.5) (layer B.Cu) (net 5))
 (segment (start 144.3 102.95) (end 145.015002 102.95) (width 0.5) (layer B.Cu) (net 5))
 (segment (start 145.3 103.8) (end 145.280001 103.780001) (width 0.5) (layer B.Cu) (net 5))
 (segment (start 147.1625 103.8) (end 145.3 103.8) (width 0.5) (layer B.Cu) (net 5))
 (segment (start 145.280001 103.214999) (end 145.280001 103.780001) (width 0.5) (layer B.Cu) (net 5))
 (segment (start 147.1625 106.1375) (end 146.9 106.4) (width 0.25) (layer B.Cu) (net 5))
 (segment (start 147.1625 103.8) (end 147.1625 106.1375) (width 0.25) (layer B.Cu) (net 5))
 (segment (start 145.280001 103.780001) (end 145.280001 104.585001) (width 0.5) (layer B.Cu) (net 5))
 (segment (start 145.015002 104.85) (end 144.3 104.85) (width 0.5) (layer B.Cu) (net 5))
 (segment (start 145.280001 104.585001) (end 145.015002 104.85) (width 0.5) (layer B.Cu) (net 5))
 (via (at 152 96.5) (size 0.8) (drill 0.4) (layers F.Cu B.Cu) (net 5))
 (segment (start 143.9625 101.3) (end 145.11251 100.14999) (width 0.5) (layer B.Cu) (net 5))
 (segment (start 146.768392 99.97501) (end 148.3 98.443402) (width 0.5) (layer B.Cu) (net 5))
 (segment (start 145.22499 99.97501) (end 146.768392 99.97501) (width 0.5) (layer B.Cu) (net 5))
 (segment (start 145.11251 100.14999) (end 145.11251 100.08749) (width 0.5) (layer B.Cu) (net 5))
 (segment (start 145.11251 100.08749) (end 145.22499 99.97501) (width 0.5) (layer B.Cu) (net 5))
 (segment (start 148.3 98.443402) (end 148.3 97.8) (width 0.5) (layer B.Cu) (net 5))
 (segment (start 149.6 96.5) (end 152 96.5) (width 0.5) (layer B.Cu) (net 5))
 (segment (start 148.3 97.8) (end 149.6 96.5) (width 0.5) (layer B.Cu) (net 5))
 (segment (start 147.85 104.9875) (end 149.0375 103.8) (width 0.25) (layer B.Cu) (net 11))
 (segment (start 147.85 106.4) (end 147.85 104.9875) (width 0.25) (layer B.Cu) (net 11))
 (via (at 150 106.1) (size 0.51) (drill 0.3) (layers F.Cu B.Cu) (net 14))
 (segment (start 150 107.458402) (end 150 106.1) (width 0.25) (layer B.Cu) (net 14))
 (segment (start 147.85 108.6) (end 148.858402 108.6) (width 0.25) (layer B.Cu) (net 14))
 (segment (start 148.858402 108.6) (end 150 107.458402) (width 0.25) (layer B.Cu) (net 14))
 (segment (start 148.85 106.1) (end 148.75 106) (width 0.25) (layer F.Cu) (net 14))
 (segment (start 150 106.1) (end 148.85 106.1) (width 0.25) (layer F.Cu) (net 14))
 (segment (start 148.855001 107.744999) (end 149.2 107.4) (width 0.25) (layer B.Cu) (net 13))
 (via (at 149.2 107.4) (size 0.51) (drill 0.3) (layers F.Cu B.Cu) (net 13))
 (segment (start 146.025001 107.744999) (end 148.855001 107.744999) (width 0.25) (layer B.Cu) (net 13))
 (segment (start 145.95 108.6) (end 145.95 107.82) (width 0.25) (layer B.Cu) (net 13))
 (segment (start 145.95 107.82) (end 146.025001 107.744999) (width 0.25) (layer B.Cu) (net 13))
 (segment (start 149.2 107.25) (end 148.75 106.8) (width 0.25) (layer F.Cu) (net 13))
 (segment (start 149.2 107.4) (end 149.2 107.25) (width 0.25) (layer F.Cu) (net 13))
 (via (at 145.65 98.45) (size 0.51) (drill 0.3) (layers F.Cu B.Cu) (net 7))
 (segment (start 145.7 99.75) (end 145.7 98.5) (width 0.25) (layer F.Cu) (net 7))
 (segment (start 145.7 98.5) (end 145.65 98.45) (width 0.25) (layer F.Cu) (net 7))
 (segment (start 145.65 97.0625) (end 145.6625 97.05) (width 0.25) (layer B.Cu) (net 7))
 (segment (start 145.65 98.45) (end 145.65 97.0625) (width 0.25) (layer B.Cu) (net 7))
 (segment (start 152.885002 102.8) (end 148.75 102.8) (width 0.25) (layer F.Cu) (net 3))
 (segment (start 153.075001 108.774999) (end 153.075001 102.989999) (width 0.25) (layer F.Cu) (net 3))
 (segment (start 153.075001 102.989999) (end 152.885002 102.8) (width 0.25) (layer F.Cu) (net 3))
 (segment (start 153 108.85) (end 153.075001 108.774999) (width 0.25) (layer F.Cu) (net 3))
 (segment (start 152 108.85) (end 153 108.85) (width 0.25) (layer F.Cu) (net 3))
 (segment (start 151.6 103.6) (end 152 104) (width 0.25) (layer F.Cu) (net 2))
 (segment (start 148.75 103.6) (end 151.6 103.6) (width 0.25) (layer F.Cu) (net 2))
 (segment (start 140.25 102) (end 141.1825 102) (width 0.25) (layer F.Cu) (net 1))
 (via (at 141.9 101.2825) (size 0.51) (drill 0.3) (layers F.Cu B.Cu) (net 1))
 (segment (start 141.1825 102) (end 141.9 101.2825) (width 0.25) (layer F.Cu) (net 1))
 (segment (start 140.5 96.5) (end 140.5 98.66) (width 0.25) (layer F.Cu) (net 1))
 (segment (start 141.9 101.2825) (end 141.3825 101.2825) (width 0.25) (layer B.Cu) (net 1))
 (segment (start 141.3825 101.2825) (end 140.65 100.55) (width 0.25) (layer B.Cu) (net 1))
 (segment (start 140.65 100.55) (end 140.65 99.75) (width 0.25) (layer B.Cu) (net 1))
 (via (at 140.25 99.35) (size 0.51) (drill 0.3) (layers F.Cu B.Cu) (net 1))
 (segment (start 140.65 99.75) (end 140.25 99.35) (width 0.25) (layer B.Cu) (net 1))
 (segment (start 140.25 98.91) (end 140.5 98.66) (width 0.25) (layer F.Cu) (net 1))
 (segment (start 140.25 99.35) (end 140.25 98.91) (width 0.25) (layer F.Cu) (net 1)))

